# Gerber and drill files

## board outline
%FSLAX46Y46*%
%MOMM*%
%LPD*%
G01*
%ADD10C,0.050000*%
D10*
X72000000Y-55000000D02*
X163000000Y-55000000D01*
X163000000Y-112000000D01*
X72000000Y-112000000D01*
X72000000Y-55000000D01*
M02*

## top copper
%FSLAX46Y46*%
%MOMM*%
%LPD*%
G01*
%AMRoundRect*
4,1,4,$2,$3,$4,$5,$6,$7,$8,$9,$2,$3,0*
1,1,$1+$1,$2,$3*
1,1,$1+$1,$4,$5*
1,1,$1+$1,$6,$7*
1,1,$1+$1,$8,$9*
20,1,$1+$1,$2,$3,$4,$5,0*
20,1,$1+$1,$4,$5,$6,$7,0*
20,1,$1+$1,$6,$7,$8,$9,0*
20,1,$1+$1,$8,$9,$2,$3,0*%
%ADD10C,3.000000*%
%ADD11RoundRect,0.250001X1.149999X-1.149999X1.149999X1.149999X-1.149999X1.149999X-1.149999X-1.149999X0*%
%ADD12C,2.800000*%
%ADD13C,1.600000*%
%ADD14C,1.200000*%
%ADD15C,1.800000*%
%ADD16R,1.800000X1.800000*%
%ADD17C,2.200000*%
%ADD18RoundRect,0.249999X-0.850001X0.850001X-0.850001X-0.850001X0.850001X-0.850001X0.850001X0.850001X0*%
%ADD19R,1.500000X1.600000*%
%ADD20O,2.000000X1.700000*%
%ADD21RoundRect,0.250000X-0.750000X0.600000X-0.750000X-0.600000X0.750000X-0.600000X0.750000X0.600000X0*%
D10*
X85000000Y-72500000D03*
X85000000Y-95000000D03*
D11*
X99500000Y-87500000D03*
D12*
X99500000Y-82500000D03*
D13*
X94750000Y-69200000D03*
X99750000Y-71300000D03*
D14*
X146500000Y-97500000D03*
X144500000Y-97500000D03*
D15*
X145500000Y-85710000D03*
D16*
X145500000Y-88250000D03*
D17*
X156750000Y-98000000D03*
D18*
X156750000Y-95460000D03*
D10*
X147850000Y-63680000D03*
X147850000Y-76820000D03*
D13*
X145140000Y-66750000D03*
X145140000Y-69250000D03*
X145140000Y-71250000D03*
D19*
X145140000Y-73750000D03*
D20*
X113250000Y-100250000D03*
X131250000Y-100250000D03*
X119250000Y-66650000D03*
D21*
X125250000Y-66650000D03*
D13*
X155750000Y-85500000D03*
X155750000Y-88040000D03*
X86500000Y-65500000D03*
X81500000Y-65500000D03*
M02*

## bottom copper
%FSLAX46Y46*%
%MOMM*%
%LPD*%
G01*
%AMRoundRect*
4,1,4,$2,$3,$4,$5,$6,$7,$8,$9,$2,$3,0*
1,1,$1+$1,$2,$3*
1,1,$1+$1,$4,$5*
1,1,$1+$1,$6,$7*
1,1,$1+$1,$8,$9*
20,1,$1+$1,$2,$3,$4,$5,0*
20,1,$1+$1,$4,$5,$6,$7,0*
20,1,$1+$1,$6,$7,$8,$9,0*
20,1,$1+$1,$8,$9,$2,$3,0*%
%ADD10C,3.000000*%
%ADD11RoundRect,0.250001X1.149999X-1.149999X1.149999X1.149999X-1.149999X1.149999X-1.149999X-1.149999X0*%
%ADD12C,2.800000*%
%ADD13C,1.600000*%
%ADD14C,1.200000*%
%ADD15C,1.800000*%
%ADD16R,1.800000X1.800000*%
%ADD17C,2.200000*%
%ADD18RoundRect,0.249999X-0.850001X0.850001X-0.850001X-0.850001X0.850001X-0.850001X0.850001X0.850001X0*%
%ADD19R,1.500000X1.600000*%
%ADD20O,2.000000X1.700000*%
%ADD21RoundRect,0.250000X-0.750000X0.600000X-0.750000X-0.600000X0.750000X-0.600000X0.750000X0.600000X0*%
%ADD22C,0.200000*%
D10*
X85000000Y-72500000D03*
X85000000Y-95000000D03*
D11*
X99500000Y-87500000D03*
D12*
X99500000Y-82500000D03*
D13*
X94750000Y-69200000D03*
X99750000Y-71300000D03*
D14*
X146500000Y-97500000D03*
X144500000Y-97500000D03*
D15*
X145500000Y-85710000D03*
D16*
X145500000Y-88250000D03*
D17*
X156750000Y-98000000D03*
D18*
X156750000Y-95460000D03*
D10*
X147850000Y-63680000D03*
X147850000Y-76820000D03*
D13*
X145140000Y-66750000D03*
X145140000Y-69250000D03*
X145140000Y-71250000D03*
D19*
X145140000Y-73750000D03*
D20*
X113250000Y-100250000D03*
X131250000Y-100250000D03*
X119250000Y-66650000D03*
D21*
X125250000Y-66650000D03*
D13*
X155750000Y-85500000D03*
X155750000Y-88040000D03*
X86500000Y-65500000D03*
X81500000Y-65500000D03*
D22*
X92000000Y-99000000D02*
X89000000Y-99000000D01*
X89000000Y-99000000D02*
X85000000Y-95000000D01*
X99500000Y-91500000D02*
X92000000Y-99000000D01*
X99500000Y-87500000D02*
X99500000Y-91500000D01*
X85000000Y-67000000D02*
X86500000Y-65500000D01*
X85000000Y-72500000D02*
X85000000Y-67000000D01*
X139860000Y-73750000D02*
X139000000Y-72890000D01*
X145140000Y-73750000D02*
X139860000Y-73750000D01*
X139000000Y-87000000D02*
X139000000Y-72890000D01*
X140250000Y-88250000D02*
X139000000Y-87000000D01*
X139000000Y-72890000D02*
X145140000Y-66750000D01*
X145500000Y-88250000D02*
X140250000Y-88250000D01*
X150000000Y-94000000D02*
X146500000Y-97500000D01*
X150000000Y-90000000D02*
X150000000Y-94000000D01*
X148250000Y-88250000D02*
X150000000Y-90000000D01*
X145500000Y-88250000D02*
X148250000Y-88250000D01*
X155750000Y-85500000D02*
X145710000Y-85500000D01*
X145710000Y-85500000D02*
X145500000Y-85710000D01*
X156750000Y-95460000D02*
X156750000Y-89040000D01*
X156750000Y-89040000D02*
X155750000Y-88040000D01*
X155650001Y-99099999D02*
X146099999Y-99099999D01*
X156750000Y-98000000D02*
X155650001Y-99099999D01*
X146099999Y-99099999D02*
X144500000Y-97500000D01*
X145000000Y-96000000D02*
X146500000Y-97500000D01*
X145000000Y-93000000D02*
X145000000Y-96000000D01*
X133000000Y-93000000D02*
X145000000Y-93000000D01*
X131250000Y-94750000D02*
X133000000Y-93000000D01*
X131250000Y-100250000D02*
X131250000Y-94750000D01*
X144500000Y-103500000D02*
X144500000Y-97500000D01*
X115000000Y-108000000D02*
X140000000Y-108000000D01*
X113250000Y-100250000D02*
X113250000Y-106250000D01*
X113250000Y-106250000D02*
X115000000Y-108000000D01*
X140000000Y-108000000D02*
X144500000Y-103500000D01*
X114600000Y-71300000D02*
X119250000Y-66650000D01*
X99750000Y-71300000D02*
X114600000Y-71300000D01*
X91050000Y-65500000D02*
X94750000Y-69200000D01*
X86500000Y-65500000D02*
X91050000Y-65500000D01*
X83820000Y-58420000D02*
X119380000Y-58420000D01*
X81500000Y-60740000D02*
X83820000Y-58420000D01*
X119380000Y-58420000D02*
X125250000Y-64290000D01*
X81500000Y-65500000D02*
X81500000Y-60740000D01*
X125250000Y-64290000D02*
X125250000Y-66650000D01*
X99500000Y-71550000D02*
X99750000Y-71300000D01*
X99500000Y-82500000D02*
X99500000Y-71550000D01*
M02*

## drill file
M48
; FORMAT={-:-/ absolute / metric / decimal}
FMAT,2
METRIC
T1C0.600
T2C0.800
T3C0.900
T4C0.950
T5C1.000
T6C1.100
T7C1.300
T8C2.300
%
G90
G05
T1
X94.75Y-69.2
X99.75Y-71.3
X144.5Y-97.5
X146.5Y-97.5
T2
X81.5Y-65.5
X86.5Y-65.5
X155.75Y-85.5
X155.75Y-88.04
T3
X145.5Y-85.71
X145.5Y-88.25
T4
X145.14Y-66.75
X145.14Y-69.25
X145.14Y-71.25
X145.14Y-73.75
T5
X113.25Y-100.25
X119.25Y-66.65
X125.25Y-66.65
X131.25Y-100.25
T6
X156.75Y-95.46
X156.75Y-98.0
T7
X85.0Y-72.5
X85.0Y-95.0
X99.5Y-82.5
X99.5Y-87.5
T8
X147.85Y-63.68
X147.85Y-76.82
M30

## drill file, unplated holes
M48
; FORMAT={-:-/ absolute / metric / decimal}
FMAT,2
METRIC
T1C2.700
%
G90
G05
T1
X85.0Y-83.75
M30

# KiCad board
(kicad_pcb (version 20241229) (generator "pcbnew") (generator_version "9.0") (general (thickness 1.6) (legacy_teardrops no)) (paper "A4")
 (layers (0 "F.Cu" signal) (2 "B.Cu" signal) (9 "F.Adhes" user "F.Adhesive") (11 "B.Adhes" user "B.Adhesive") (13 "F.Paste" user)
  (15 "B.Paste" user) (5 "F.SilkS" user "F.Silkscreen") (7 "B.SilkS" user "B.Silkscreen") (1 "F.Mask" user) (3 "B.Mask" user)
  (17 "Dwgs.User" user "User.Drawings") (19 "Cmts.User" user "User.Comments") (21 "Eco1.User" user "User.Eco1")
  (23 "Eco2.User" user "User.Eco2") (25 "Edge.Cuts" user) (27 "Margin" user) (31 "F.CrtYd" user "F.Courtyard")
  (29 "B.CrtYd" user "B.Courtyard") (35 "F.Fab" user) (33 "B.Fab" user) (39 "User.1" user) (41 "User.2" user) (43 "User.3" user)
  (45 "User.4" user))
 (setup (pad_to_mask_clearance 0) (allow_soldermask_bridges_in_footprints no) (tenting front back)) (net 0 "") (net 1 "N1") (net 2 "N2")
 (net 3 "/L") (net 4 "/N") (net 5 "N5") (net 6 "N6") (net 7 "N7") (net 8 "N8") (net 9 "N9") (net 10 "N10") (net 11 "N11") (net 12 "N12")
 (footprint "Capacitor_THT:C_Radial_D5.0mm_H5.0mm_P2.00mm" (layer "F.Cu") (at 144.5 97.5)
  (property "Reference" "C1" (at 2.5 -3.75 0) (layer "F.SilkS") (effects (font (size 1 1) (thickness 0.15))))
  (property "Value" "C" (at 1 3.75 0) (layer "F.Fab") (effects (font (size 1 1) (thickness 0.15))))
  (pad "1" thru_hole circle (at 0 0) (size 1.2 1.2) (drill 0.6) (layers "*.Cu" "*.Mask") (remove_unused_layers no) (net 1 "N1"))
  (pad "2" thru_hole circle (at 2 0) (size 1.2 1.2) (drill 0.6) (layers "*.Cu" "*.Mask") (remove_unused_layers no) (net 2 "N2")))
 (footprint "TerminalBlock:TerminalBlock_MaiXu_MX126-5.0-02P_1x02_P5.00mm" (layer "F.Cu") (at 99.5 87.5 90)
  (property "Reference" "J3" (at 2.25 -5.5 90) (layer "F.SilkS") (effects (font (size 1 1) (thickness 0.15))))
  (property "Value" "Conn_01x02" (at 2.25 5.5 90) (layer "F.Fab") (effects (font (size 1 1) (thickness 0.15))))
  (pad "1" thru_hole roundrect (at 0 0 90) (size 2.8 2.8) (drill 1.3) (layers "*.Cu" "*.Mask") (remove_unused_layers no)
   (roundrect_rratio 0.089286) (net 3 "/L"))
  (pad "2" thru_hole circle (at 5 0 90) (size 2.8 2.8) (drill 1.3) (layers "*.Cu" "*.Mask") (remove_unused_layers no) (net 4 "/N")))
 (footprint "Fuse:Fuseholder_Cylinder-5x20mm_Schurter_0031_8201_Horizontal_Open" (layer "F.Cu") (at 85 72.5 -90)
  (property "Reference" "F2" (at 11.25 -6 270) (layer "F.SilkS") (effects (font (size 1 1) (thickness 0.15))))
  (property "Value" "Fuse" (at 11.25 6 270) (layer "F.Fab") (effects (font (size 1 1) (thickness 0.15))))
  (pad "" np_thru_hole circle (at 11.25 0 270) (size 2.7 2.7) (drill 2.7) (layers "*.Cu" "*.Mask"))
  (pad "1" thru_hole circle (at 0 0 270) (size 3 3) (drill 1.3) (layers "*.Cu" "*.Mask") (remove_unused_layers no) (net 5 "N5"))
  (pad "2" thru_hole circle (at 22.5 0 270) (size 3 3) (drill 1.3) (layers "*.Cu" "*.Mask") (remove_unused_layers no) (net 3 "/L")))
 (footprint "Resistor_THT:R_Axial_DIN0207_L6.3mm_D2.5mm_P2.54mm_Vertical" (layer "F.Cu") (at 155.75 88.04 90)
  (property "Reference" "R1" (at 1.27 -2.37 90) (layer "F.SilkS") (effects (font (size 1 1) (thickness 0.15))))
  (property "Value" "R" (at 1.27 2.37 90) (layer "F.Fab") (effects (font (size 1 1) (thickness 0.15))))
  (pad "1" thru_hole circle (at 0 0 90) (size 1.6 1.6) (drill 0.8) (layers "*.Cu" "*.Mask") (remove_unused_layers no) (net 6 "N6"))
  (pad "2" thru_hole circle (at 2.54 0 90) (size 1.6 1.6) (drill 0.8) (layers "*.Cu" "*.Mask") (remove_unused_layers no) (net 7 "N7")))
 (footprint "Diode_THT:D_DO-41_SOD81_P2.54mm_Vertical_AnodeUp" (layer "F.Cu") (at 156.75 95.46 -90)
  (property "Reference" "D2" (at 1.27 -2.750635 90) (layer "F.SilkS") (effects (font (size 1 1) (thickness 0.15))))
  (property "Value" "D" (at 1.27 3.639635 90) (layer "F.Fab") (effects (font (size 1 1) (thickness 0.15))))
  (pad "1" thru_hole roundrect (at 0 0 270) (size 2.2 2.2) (drill 1.1) (layers "*.Cu" "*.Mask") (remove_unused_layers no)
   (roundrect_rratio 0.113636) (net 6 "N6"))
  (pad "2" thru_hole circle (at 2.54 0 270) (size 2.2 2.2) (drill 1.1) (layers "*.Cu" "*.Mask") (remove_unused_layers no) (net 1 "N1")))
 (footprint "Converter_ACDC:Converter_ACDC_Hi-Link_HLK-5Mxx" (layer "F.Cu") (at 125.25 66.65 -90)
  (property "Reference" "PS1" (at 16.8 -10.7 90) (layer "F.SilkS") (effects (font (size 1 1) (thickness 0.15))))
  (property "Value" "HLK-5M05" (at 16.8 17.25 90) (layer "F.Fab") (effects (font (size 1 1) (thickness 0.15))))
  (pad "1" thru_hole roundrect (at 0 0 270) (size 1.7 2) (drill 1) (layers "*.Cu" "*.Mask") (remove_unused_layers no)
   (roundrect_rratio 0.147059) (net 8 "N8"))
  (pad "2" thru_hole oval (at 0 6 270) (size 1.7 2) (drill 1) (layers "*.Cu" "*.Mask") (remove_unused_layers no) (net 4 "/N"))
  (pad "3" thru_hole oval (at 33.6 -6 270) (size 1.7 2) (drill 1) (layers "*.Cu" "*.Mask") (remove_unused_layers no) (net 2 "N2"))
  (pad "4" thru_hole oval (at 33.6 12 270) (size 1.7 2) (drill 1) (layers "*.Cu" "*.Mask") (remove_unused_layers no) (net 1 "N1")))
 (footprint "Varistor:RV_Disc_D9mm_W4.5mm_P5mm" (layer "F.Cu") (at 94.75 69.2)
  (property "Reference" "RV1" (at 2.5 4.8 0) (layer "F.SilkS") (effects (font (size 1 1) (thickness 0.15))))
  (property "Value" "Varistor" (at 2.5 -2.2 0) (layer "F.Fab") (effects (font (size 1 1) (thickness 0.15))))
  (pad "1" thru_hole circle (at 0 0) (size 1.6 1.6) (drill 0.6) (layers "*.Cu" "*.Mask") (remove_unused_layers no) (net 5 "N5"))
  (pad "2" thru_hole circle (at 5 2.1) (size 1.6 1.6) (drill 0.6) (layers "*.Cu" "*.Mask") (remove_unused_layers no) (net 4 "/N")))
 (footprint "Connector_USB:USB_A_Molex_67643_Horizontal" (layer "F.Cu") (at 145.14 73.75 90)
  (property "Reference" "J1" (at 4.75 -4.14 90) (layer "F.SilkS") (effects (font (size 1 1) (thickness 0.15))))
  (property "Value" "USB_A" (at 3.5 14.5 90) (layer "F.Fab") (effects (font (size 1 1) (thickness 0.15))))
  (pad "1" thru_hole rect (at 0 0 90) (size 1.6 1.5) (drill 0.95) (layers "*.Cu" "*.Mask") (remove_unused_layers no) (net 2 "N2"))
  (pad "2" thru_hole circle (at 2.5 0 90) (size 1.6 1.6) (drill 0.95) (layers "*.Cu" "*.Mask") (remove_unused_layers no) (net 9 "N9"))
  (pad "3" thru_hole circle (at 4.5 0 90) (size 1.6 1.6) (drill 0.95) (layers "*.Cu" "*.Mask") (remove_unused_layers no) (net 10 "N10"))
  (pad "4" thru_hole circle (at 7 0 90) (size 1.6 1.6) (drill 0.95) (layers "*.Cu" "*.Mask") (remove_unused_layers no) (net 2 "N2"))
  (pad "5" thru_hole circle (at -3.07 2.71 90) (size 3 3) (drill 2.3) (layers "*.Cu" "*.Mask") (remove_unused_layers no) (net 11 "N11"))
  (pad "5" thru_hole circle (at 10.07 2.71 90) (size 3 3) (drill 2.3) (layers "*.Cu" "*.Mask") (remove_unused_layers no) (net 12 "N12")))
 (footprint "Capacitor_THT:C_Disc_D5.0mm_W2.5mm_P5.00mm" (layer "F.Cu") (at 81.5 65.5)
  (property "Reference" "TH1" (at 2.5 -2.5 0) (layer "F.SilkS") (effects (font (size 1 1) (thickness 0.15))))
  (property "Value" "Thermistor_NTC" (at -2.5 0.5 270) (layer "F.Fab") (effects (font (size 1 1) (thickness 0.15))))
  (pad "1" thru_hole circle (at 0 0) (size 1.6 1.6) (drill 0.8) (layers "*.Cu" "*.Mask") (remove_unused_layers no) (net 8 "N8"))
  (pad "2" thru_hole circle (at 5 0) (size 1.6 1.6) (drill 0.8) (layers "*.Cu" "*.Mask") (remove_unused_layers no) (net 5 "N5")))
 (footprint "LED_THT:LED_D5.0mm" (layer "F.Cu") (at 145.5 88.25 90)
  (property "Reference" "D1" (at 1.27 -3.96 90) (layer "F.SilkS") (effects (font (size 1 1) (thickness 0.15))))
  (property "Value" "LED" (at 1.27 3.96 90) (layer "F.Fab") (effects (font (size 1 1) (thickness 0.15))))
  (pad "1" thru_hole rect (at 0 0 90) (size 1.8 1.8) (drill 0.9) (layers "*.Cu" "*.Mask") (remove_unused_layers no) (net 2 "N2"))
  (pad "2" thru_hole circle (at 2.54 0 90) (size 1.8 1.8) (drill 0.9) (layers "*.Cu" "*.Mask") (remove_unused_layers no) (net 7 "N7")))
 (gr_rect (start 72 55) (end 163 112) (stroke (width 0.05) (type default)) (fill no) (layer "Edge.Cuts"))
 (segment (start 113.25 106.25) (end 115 108) (width 0.2) (layer "B.Cu") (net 1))
 (segment (start 146.099999 99.099999) (end 144.5 97.5) (width 0.2) (layer "B.Cu") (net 1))
 (segment (start 115 108) (end 140 108) (width 0.2) (layer "B.Cu") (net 1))
 (segment (start 113.25 100.25) (end 113.25 106.25) (width 0.2) (layer "B.Cu") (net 1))
 (segment (start 155.650001 99.099999) (end 146.099999 99.099999) (width 0.2) (layer "B.Cu") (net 1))
 (segment (start 156.75 98) (end 155.650001 99.099999) (width 0.2) (layer "B.Cu") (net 1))
 (segment (start 144.5 103.5) (end 144.5 97.5) (width 0.2) (layer "B.Cu") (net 1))
 (segment (start 140 108) (end 144.5 103.5) (width 0.2) (layer "B.Cu") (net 1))
 (segment (start 139.86 73.75) (end 139 72.89) (width 0.2) (layer "B.Cu") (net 2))
 (segment (start 150 90) (end 150 94) (width 0.2) (layer "B.Cu") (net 2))
 (segment (start 139 87) (end 139 72.89) (width 0.2) (layer "B.Cu") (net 2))
 (segment (start 139 72.89) (end 145.14 66.75) (width 0.2) (layer "B.Cu") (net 2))
 (segment (start 131.25 100.25) (end 131.25 94.75) (width 0.2) (layer "B.Cu") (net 2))
 (segment (start 145 93) (end 145 96) (width 0.2) (layer "B.Cu") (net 2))
 (segment (start 145 96) (end 146.5 97.5) (width 0.2) (layer "B.Cu") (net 2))
 (segment (start 148.25 88.25) (end 150 90) (width 0.2) (layer "B.Cu") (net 2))
 (segment (start 145.14 73.75) (end 139.86 73.75) (width 0.2) (layer "B.Cu") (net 2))
 (segment (start 145.5 88.25) (end 140.25 88.25) (width 0.2) (layer "B.Cu") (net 2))
 (segment (start 145.5 88.25) (end 148.25 88.25) (width 0.2) (layer "B.Cu") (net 2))
 (segment (start 133 93) (end 145 93) (width 0.2) (layer "B.Cu") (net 2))
 (segment (start 131.25 94.75) (end 133 93) (width 0.2) (layer "B.Cu") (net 2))
 (segment (start 150 94) (end 146.5 97.5) (width 0.2) (layer "B.Cu") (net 2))
 (segment (start 140.25 88.25) (end 139 87) (width 0.2) (layer "B.Cu") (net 2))
 (segment (start 155.75 85.5) (end 145.71 85.5) (width 0.2) (layer "B.Cu") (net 7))
 (segment (start 145.71 85.5) (end 145.5 85.71) (width 0.2) (layer "B.Cu") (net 7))
 (segment (start 156.75 89.04) (end 155.75 88.04) (width 0.2) (layer "B.Cu") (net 6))
 (segment (start 156.75 95.46) (end 156.75 89.04) (width 0.2) (layer "B.Cu") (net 6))
 (segment (start 92 99) (end 89 99) (width 0.2) (layer "B.Cu") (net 3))
 (segment (start 99.5 87.5) (end 99.5 91.5) (width 0.2) (layer "B.Cu") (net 3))
 (segment (start 89 99) (end 85 95) (width 0.2) (layer "B.Cu") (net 3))
 (segment (start 99.5 91.5) (end 92 99) (width 0.2) (layer "B.Cu") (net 3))
 (segment (start 99.5 82.5) (end 99.5 71.55) (width 0.2) (layer "B.Cu") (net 4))
 (segment (start 99.5 71.55) (end 99.75 71.3) (width 0.2) (layer "B.Cu") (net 4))
 (segment (start 114.6 71.3) (end 119.25 66.65) (width 0.2) (layer "B.Cu") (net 4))
 (segment (start 99.75 71.3) (end 114.6 71.3) (width 0.2) (layer "B.Cu") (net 4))
 (segment (start 125.25 64.29) (end 125.25 66.65) (width 0.2) (layer "B.Cu") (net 8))
 (segment (start 81.5 65.5) (end 81.5 60.74) (width 0.2) (layer "B.Cu") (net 8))
 (segment (start 81.5 60.74) (end 83.82 58.42) (width 0.2) (layer "B.Cu") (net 8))
 (segment (start 83.82 58.42) (end 119.38 58.42) (width 0.2) (layer "B.Cu") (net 8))
 (segment (start 119.38 58.42) (end 125.25 64.29) (width 0.2) (layer "B.Cu") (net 8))
 (segment (start 91.05 65.5) (end 94.75 69.2) (width 0.2) (layer "B.Cu") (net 5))
 (segment (start 86.5 65.5) (end 91.05 65.5) (width 0.2) (layer "B.Cu") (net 5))
 (segment (start 85 67) (end 86.5 65.5) (width 0.2) (layer "B.Cu") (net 5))
 (segment (start 85 72.5) (end 85 67) (width 0.2) (layer "B.Cu") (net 5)))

